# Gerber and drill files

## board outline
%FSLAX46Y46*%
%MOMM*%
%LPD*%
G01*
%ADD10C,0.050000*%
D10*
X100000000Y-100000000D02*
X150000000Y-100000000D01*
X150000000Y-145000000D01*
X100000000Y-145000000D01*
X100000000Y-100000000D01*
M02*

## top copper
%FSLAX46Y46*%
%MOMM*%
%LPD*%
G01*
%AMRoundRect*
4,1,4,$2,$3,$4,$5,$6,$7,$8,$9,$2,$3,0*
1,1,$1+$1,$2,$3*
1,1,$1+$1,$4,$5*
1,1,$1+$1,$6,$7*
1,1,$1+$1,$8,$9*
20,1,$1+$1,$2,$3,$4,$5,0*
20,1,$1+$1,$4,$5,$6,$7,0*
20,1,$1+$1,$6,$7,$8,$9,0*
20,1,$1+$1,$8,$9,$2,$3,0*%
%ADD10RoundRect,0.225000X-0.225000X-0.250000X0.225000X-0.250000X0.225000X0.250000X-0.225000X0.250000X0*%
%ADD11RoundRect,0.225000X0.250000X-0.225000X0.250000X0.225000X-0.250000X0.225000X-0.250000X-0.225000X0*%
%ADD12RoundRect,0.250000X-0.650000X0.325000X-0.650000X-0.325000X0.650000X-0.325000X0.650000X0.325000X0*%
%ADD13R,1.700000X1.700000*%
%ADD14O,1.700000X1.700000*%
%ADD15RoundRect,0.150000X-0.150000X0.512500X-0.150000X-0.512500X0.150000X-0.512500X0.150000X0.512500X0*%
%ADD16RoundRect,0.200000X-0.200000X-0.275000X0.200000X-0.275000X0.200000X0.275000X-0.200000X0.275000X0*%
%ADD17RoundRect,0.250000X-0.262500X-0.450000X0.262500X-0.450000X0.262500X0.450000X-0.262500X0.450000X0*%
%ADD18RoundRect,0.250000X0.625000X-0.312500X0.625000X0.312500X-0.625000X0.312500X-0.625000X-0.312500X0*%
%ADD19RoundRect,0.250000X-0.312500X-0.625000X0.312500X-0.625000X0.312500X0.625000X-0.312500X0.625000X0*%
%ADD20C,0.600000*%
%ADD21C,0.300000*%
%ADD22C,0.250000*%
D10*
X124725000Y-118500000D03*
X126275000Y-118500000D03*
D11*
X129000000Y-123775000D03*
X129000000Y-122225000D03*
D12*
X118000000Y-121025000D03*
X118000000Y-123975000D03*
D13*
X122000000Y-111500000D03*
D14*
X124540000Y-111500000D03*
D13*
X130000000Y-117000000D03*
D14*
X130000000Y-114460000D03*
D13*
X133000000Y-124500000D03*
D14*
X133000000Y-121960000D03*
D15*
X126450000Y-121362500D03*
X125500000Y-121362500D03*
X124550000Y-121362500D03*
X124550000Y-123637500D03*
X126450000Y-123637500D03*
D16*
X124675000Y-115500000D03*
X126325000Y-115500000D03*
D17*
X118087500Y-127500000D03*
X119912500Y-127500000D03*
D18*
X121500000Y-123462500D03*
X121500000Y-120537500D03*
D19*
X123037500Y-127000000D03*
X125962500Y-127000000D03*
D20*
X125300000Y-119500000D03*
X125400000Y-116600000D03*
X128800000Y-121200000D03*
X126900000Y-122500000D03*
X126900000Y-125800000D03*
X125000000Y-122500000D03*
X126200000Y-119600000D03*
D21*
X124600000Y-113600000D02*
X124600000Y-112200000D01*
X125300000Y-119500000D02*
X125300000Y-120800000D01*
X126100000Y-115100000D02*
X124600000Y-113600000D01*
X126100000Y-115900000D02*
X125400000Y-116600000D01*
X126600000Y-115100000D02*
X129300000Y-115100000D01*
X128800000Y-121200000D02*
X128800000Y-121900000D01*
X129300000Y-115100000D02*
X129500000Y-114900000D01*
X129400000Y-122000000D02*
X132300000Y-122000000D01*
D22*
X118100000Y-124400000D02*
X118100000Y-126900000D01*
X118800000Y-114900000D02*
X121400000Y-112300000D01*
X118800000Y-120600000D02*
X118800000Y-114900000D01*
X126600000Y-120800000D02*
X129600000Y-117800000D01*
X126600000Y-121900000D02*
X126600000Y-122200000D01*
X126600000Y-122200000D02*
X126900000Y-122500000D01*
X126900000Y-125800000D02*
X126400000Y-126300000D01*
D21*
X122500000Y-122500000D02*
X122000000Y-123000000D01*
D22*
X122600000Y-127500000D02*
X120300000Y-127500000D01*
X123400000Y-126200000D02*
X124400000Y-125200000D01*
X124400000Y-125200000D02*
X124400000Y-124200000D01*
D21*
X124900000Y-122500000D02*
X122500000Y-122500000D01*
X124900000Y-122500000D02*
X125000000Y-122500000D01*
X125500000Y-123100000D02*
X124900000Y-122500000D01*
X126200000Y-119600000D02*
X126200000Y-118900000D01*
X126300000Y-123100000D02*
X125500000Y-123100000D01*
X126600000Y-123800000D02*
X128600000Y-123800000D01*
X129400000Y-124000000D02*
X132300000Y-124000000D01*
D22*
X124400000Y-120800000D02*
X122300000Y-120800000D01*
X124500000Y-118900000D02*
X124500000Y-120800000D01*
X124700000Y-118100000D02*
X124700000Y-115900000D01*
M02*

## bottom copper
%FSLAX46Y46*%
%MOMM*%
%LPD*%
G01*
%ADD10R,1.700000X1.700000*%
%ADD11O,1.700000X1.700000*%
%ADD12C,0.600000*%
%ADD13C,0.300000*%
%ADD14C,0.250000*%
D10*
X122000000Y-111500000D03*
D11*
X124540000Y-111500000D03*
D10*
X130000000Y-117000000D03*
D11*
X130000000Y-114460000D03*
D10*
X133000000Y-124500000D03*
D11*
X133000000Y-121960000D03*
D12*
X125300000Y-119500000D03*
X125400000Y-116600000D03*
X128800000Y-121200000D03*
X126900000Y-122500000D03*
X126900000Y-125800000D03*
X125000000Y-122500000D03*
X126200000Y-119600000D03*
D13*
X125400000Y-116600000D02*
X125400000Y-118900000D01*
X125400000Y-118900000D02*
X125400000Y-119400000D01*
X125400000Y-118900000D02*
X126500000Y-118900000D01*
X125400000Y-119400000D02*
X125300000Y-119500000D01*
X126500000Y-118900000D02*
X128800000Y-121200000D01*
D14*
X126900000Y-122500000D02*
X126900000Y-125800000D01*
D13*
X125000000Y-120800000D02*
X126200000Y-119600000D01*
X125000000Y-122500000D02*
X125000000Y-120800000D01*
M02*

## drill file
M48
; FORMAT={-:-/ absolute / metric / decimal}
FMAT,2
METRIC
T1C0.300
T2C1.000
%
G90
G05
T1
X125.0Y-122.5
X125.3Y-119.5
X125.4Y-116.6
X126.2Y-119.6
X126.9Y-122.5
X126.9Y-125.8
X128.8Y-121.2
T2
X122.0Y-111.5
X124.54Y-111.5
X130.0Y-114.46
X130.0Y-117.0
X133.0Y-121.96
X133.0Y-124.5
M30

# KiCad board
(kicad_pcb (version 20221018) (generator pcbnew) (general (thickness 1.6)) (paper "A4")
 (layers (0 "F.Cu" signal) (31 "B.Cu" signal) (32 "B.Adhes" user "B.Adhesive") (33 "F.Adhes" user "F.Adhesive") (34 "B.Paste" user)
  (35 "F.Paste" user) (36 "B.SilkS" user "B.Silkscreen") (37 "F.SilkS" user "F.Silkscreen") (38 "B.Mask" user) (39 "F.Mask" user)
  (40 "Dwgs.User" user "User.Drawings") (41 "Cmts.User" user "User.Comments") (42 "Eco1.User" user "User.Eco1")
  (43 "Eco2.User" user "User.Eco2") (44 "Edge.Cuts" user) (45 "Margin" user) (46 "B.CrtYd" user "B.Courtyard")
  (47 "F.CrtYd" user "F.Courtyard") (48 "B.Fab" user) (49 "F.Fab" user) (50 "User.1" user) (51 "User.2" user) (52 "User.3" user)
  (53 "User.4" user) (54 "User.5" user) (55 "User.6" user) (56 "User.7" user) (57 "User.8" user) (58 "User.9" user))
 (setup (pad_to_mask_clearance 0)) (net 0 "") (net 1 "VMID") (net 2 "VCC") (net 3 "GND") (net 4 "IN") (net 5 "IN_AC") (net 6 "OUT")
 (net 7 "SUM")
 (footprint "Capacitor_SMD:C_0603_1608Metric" (layer "F.Cu") (at 125.5 118.5)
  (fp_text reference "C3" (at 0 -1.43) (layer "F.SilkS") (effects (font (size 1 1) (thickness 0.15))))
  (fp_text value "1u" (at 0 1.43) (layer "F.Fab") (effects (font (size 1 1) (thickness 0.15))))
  (pad "1" smd roundrect (at -0.775 0) (size 0.9 0.95) (layers "F.Cu" "F.Paste" "F.Mask") (roundrect_rratio 0.25) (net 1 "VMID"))
  (pad "2" smd roundrect (at 0.775 0) (size 0.9 0.95) (layers "F.Cu" "F.Paste" "F.Mask") (roundrect_rratio 0.25) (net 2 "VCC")))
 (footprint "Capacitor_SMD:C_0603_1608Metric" (layer "F.Cu") (at 129 123 90)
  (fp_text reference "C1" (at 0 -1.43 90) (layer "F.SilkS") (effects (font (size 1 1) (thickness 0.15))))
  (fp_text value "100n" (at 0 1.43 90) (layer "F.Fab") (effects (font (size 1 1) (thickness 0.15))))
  (pad "1" smd roundrect (at -0.775 0 90) (size 0.9 0.95) (layers "F.Cu" "F.Paste" "F.Mask") (roundrect_rratio 0.25) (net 2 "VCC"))
  (pad "2" smd roundrect (at 0.775 0 90) (size 0.9 0.95) (layers "F.Cu" "F.Paste" "F.Mask") (roundrect_rratio 0.25) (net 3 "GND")))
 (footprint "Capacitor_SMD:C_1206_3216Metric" (layer "F.Cu") (at 118 122.5 -90)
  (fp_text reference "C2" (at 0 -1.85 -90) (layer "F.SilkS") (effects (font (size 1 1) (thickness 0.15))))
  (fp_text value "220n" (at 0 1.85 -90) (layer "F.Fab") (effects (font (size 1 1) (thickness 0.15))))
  (pad "1" smd roundrect (at -1.475 0 270) (size 1.15 1.8) (layers "F.Cu" "F.Paste" "F.Mask") (roundrect_rratio 0.217391) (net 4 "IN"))
  (pad "2" smd roundrect (at 1.475 0 270) (size 1.15 1.8) (layers "F.Cu" "F.Paste" "F.Mask") (roundrect_rratio 0.217391) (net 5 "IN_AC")))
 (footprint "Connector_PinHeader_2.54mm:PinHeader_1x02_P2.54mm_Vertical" (layer "F.Cu") (at 122 111.5 90)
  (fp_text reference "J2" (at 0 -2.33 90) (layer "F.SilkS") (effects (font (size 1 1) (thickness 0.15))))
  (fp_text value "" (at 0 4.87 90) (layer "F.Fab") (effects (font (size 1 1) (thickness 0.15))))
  (pad "1" thru_hole rect (at 0 0 90) (size 1.7 1.7) (drill 1) (layers "*.Cu" "*.Mask") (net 4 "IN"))
  (pad "2" thru_hole oval (at 0 2.54 90) (size 1.7 1.7) (drill 1) (layers "*.Cu" "*.Mask") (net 3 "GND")))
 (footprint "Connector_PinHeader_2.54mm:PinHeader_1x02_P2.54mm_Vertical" (layer "F.Cu") (at 130 117 180)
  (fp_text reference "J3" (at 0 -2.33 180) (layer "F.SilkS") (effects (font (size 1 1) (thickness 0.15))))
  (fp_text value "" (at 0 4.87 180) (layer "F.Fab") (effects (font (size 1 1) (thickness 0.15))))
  (pad "1" thru_hole rect (at 0 0 180) (size 1.7 1.7) (drill 1) (layers "*.Cu" "*.Mask") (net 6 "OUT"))
  (pad "2" thru_hole oval (at 0 2.54 180) (size 1.7 1.7) (drill 1) (layers "*.Cu" "*.Mask") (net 3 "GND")))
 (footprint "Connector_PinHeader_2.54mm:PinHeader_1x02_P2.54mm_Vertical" (layer "F.Cu") (at 133 124.5 180)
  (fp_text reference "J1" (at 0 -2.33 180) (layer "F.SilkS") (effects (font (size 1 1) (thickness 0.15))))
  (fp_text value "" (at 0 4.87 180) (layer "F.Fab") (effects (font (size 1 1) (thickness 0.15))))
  (pad "1" thru_hole rect (at 0 0 180) (size 1.7 1.7) (drill 1) (layers "*.Cu" "*.Mask") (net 2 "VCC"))
  (pad "2" thru_hole oval (at 0 2.54 180) (size 1.7 1.7) (drill 1) (layers "*.Cu" "*.Mask") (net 3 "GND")))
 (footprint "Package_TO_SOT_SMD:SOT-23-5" (layer "F.Cu") (at 125.5 122.5 -90)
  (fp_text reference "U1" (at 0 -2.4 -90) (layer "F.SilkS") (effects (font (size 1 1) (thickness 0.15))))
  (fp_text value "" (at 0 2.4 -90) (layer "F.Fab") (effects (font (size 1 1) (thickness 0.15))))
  (pad "1" smd roundrect (at -1.1375 -0.95 270) (size 1.325 0.6) (layers "F.Cu" "F.Paste" "F.Mask") (roundrect_rratio 0.25) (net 6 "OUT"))
  (pad "2" smd roundrect (at -1.1375 0 270) (size 1.325 0.6) (layers "F.Cu" "F.Paste" "F.Mask") (roundrect_rratio 0.25) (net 3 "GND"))
  (pad "3" smd roundrect (at -1.1375 0.95 270) (size 1.325 0.6) (layers "F.Cu" "F.Paste" "F.Mask") (roundrect_rratio 0.25) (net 1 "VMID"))
  (pad "4" smd roundrect (at 1.1375 0.95 270) (size 1.325 0.6) (layers "F.Cu" "F.Paste" "F.Mask") (roundrect_rratio 0.25) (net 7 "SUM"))
  (pad "5" smd roundrect (at 1.1375 -0.95 270) (size 1.325 0.6) (layers "F.Cu" "F.Paste" "F.Mask") (roundrect_rratio 0.25) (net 2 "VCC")))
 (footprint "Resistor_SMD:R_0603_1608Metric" (layer "F.Cu") (at 125.5 115.5)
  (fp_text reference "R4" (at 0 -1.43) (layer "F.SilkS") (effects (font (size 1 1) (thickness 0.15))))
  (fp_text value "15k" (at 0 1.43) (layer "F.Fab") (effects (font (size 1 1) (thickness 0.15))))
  (pad "1" smd roundrect (at -0.825 0) (size 0.8 0.95) (layers "F.Cu" "F.Paste" "F.Mask") (roundrect_rratio 0.25) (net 1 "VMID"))
  (pad "2" smd roundrect (at 0.825 0) (size 0.8 0.95) (layers "F.Cu" "F.Paste" "F.Mask") (roundrect_rratio 0.25) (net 3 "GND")))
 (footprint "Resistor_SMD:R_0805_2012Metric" (layer "F.Cu") (at 119 127.5)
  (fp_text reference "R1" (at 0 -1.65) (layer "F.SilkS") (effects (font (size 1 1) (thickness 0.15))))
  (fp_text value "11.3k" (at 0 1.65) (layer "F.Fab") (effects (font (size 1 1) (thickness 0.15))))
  (pad "1" smd roundrect (at -0.9125 0) (size 1.025 1.4) (layers "F.Cu" "F.Paste" "F.Mask") (roundrect_rratio 0.243902) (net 5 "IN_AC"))
  (pad "2" smd roundrect (at 0.9125 0) (size 1.025 1.4) (layers "F.Cu" "F.Paste" "F.Mask") (roundrect_rratio 0.243902) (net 7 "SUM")))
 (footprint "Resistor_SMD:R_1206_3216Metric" (layer "F.Cu") (at 121.5 122 90)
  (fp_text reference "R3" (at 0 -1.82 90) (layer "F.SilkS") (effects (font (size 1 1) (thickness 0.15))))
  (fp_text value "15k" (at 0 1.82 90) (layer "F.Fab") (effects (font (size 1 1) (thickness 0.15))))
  (pad "1" smd roundrect (at -1.4625 0 90) (size 1.125 1.75) (layers "F.Cu" "F.Paste" "F.Mask") (roundrect_rratio 0.222222) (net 2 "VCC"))
  (pad "2" smd roundrect (at 1.4625 0 90) (size 1.125 1.75) (layers "F.Cu" "F.Paste" "F.Mask") (roundrect_rratio 0.222222) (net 1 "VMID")))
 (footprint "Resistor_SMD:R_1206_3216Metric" (layer "F.Cu") (at 124.5 127)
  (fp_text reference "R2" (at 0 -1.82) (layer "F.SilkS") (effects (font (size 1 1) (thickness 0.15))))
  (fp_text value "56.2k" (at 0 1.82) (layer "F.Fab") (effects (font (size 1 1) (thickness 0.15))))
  (pad "1" smd roundrect (at -1.4625 0) (size 1.125 1.75) (layers "F.Cu" "F.Paste" "F.Mask") (roundrect_rratio 0.222222) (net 7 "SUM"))
  (pad "2" smd roundrect (at 1.4625 0) (size 1.125 1.75) (layers "F.Cu" "F.Paste" "F.Mask") (roundrect_rratio 0.222222) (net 6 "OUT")))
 (gr_rect (start 100 100) (end 150 145) (stroke (width 0.05) (type default)) (fill none) (layer "Edge.Cuts"))
 (segment (start 124.6 113.6) (end 124.6 112.2) (width 0.3) (layer "F.Cu") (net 3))
 (segment (start 125.3 119.5) (end 125.3 120.8) (width 0.3) (layer "F.Cu") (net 3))
 (segment (start 126.1 115.1) (end 124.6 113.6) (width 0.3) (layer "F.Cu") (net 3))
 (segment (start 126.1 115.9) (end 125.4 116.6) (width 0.3) (layer "F.Cu") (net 3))
 (segment (start 126.6 115.1) (end 129.3 115.1) (width 0.3) (layer "F.Cu") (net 3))
 (segment (start 128.8 121.2) (end 128.8 121.9) (width 0.3) (layer "F.Cu") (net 3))
 (segment (start 129.3 115.1) (end 129.5 114.9) (width 0.3) (layer "F.Cu") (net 3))
 (segment (start 129.4 122) (end 132.3 122) (width 0.3) (layer "F.Cu") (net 3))
 (via (at 125.3 119.5) (size 0.6) (drill 0.3) (layers "F.Cu" "B.Cu") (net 3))
 (via (at 125.4 116.6) (size 0.6) (drill 0.3) (layers "F.Cu" "B.Cu") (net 3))
 (via (at 128.8 121.2) (size 0.6) (drill 0.3) (layers "F.Cu" "B.Cu") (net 3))
 (segment (start 118.1 124.4) (end 118.1 126.9) (width 0.25) (layer "F.Cu") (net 5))
 (segment (start 118.8 114.9) (end 121.4 112.3) (width 0.25) (layer "F.Cu") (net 4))
 (segment (start 118.8 120.6) (end 118.8 114.9) (width 0.25) (layer "F.Cu") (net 4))
 (segment (start 125.4 116.6) (end 125.4 118.9) (width 0.3) (layer "B.Cu") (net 3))
 (segment (start 125.4 118.9) (end 125.4 119.4) (width 0.3) (layer "B.Cu") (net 3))
 (segment (start 125.4 118.9) (end 126.5 118.9) (width 0.3) (layer "B.Cu") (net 3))
 (segment (start 125.4 119.4) (end 125.3 119.5) (width 0.3) (layer "B.Cu") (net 3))
 (segment (start 126.5 118.9) (end 128.8 121.2) (width 0.3) (layer "B.Cu") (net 3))
 (segment (start 126.6 120.8) (end 129.6 117.8) (width 0.25) (layer "F.Cu") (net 6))
 (segment (start 126.6 121.9) (end 126.6 122.2) (width 0.25) (layer "F.Cu") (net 6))
 (segment (start 126.6 122.2) (end 126.9 122.5) (width 0.25) (layer "F.Cu") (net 6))
 (segment (start 126.9 125.8) (end 126.4 126.3) (width 0.25) (layer "F.Cu") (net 6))
 (via (at 126.9 122.5) (size 0.6) (drill 0.3) (layers "F.Cu" "B.Cu") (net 6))
 (via (at 126.9 125.8) (size 0.6) (drill 0.3) (layers "F.Cu" "B.Cu") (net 6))
 (segment (start 122.5 122.5) (end 122 123) (width 0.3) (layer "F.Cu") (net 2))
 (segment (start 122.6 127.5) (end 120.3 127.5) (width 0.25) (layer "F.Cu") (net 7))
 (segment (start 123.4 126.2) (end 124.4 125.2) (width 0.25) (layer "F.Cu") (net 7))
 (segment (start 124.4 125.2) (end 124.4 124.2) (width 0.25) (layer "F.Cu") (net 7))
 (segment (start 124.9 122.5) (end 122.5 122.5) (width 0.3) (layer "F.Cu") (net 2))
 (segment (start 124.9 122.5) (end 125 122.5) (width 0.3) (layer "F.Cu") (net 2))
 (segment (start 125.5 123.1) (end 124.9 122.5) (width 0.3) (layer "F.Cu") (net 2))
 (segment (start 126.2 119.6) (end 126.2 118.9) (width 0.3) (layer "F.Cu") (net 2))
 (segment (start 126.3 123.1) (end 125.5 123.1) (width 0.3) (layer "F.Cu") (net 2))
 (segment (start 126.6 123.8) (end 128.6 123.8) (width 0.3) (layer "F.Cu") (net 2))
 (segment (start 126.9 122.5) (end 126.9 125.8) (width 0.25) (layer "B.Cu") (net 6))
 (segment (start 129.4 124) (end 132.3 124) (width 0.3) (layer "F.Cu") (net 2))
 (via (at 125 122.5) (size 0.6) (drill 0.3) (layers "F.Cu" "B.Cu") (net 2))
 (via (at 126.2 119.6) (size 0.6) (drill 0.3) (layers "F.Cu" "B.Cu") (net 2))
 (segment (start 124.4 120.8) (end 122.3 120.8) (width 0.25) (layer "F.Cu") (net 1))
 (segment (start 124.5 118.9) (end 124.5 120.8) (width 0.25) (layer "F.Cu") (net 1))
 (segment (start 124.7 118.1) (end 124.7 115.9) (width 0.25) (layer "F.Cu") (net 1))
 (segment (start 125 120.8) (end 126.2 119.6) (width 0.3) (layer "B.Cu") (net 2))
 (segment (start 125 122.5) (end 125 120.8) (width 0.3) (layer "B.Cu") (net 2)))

